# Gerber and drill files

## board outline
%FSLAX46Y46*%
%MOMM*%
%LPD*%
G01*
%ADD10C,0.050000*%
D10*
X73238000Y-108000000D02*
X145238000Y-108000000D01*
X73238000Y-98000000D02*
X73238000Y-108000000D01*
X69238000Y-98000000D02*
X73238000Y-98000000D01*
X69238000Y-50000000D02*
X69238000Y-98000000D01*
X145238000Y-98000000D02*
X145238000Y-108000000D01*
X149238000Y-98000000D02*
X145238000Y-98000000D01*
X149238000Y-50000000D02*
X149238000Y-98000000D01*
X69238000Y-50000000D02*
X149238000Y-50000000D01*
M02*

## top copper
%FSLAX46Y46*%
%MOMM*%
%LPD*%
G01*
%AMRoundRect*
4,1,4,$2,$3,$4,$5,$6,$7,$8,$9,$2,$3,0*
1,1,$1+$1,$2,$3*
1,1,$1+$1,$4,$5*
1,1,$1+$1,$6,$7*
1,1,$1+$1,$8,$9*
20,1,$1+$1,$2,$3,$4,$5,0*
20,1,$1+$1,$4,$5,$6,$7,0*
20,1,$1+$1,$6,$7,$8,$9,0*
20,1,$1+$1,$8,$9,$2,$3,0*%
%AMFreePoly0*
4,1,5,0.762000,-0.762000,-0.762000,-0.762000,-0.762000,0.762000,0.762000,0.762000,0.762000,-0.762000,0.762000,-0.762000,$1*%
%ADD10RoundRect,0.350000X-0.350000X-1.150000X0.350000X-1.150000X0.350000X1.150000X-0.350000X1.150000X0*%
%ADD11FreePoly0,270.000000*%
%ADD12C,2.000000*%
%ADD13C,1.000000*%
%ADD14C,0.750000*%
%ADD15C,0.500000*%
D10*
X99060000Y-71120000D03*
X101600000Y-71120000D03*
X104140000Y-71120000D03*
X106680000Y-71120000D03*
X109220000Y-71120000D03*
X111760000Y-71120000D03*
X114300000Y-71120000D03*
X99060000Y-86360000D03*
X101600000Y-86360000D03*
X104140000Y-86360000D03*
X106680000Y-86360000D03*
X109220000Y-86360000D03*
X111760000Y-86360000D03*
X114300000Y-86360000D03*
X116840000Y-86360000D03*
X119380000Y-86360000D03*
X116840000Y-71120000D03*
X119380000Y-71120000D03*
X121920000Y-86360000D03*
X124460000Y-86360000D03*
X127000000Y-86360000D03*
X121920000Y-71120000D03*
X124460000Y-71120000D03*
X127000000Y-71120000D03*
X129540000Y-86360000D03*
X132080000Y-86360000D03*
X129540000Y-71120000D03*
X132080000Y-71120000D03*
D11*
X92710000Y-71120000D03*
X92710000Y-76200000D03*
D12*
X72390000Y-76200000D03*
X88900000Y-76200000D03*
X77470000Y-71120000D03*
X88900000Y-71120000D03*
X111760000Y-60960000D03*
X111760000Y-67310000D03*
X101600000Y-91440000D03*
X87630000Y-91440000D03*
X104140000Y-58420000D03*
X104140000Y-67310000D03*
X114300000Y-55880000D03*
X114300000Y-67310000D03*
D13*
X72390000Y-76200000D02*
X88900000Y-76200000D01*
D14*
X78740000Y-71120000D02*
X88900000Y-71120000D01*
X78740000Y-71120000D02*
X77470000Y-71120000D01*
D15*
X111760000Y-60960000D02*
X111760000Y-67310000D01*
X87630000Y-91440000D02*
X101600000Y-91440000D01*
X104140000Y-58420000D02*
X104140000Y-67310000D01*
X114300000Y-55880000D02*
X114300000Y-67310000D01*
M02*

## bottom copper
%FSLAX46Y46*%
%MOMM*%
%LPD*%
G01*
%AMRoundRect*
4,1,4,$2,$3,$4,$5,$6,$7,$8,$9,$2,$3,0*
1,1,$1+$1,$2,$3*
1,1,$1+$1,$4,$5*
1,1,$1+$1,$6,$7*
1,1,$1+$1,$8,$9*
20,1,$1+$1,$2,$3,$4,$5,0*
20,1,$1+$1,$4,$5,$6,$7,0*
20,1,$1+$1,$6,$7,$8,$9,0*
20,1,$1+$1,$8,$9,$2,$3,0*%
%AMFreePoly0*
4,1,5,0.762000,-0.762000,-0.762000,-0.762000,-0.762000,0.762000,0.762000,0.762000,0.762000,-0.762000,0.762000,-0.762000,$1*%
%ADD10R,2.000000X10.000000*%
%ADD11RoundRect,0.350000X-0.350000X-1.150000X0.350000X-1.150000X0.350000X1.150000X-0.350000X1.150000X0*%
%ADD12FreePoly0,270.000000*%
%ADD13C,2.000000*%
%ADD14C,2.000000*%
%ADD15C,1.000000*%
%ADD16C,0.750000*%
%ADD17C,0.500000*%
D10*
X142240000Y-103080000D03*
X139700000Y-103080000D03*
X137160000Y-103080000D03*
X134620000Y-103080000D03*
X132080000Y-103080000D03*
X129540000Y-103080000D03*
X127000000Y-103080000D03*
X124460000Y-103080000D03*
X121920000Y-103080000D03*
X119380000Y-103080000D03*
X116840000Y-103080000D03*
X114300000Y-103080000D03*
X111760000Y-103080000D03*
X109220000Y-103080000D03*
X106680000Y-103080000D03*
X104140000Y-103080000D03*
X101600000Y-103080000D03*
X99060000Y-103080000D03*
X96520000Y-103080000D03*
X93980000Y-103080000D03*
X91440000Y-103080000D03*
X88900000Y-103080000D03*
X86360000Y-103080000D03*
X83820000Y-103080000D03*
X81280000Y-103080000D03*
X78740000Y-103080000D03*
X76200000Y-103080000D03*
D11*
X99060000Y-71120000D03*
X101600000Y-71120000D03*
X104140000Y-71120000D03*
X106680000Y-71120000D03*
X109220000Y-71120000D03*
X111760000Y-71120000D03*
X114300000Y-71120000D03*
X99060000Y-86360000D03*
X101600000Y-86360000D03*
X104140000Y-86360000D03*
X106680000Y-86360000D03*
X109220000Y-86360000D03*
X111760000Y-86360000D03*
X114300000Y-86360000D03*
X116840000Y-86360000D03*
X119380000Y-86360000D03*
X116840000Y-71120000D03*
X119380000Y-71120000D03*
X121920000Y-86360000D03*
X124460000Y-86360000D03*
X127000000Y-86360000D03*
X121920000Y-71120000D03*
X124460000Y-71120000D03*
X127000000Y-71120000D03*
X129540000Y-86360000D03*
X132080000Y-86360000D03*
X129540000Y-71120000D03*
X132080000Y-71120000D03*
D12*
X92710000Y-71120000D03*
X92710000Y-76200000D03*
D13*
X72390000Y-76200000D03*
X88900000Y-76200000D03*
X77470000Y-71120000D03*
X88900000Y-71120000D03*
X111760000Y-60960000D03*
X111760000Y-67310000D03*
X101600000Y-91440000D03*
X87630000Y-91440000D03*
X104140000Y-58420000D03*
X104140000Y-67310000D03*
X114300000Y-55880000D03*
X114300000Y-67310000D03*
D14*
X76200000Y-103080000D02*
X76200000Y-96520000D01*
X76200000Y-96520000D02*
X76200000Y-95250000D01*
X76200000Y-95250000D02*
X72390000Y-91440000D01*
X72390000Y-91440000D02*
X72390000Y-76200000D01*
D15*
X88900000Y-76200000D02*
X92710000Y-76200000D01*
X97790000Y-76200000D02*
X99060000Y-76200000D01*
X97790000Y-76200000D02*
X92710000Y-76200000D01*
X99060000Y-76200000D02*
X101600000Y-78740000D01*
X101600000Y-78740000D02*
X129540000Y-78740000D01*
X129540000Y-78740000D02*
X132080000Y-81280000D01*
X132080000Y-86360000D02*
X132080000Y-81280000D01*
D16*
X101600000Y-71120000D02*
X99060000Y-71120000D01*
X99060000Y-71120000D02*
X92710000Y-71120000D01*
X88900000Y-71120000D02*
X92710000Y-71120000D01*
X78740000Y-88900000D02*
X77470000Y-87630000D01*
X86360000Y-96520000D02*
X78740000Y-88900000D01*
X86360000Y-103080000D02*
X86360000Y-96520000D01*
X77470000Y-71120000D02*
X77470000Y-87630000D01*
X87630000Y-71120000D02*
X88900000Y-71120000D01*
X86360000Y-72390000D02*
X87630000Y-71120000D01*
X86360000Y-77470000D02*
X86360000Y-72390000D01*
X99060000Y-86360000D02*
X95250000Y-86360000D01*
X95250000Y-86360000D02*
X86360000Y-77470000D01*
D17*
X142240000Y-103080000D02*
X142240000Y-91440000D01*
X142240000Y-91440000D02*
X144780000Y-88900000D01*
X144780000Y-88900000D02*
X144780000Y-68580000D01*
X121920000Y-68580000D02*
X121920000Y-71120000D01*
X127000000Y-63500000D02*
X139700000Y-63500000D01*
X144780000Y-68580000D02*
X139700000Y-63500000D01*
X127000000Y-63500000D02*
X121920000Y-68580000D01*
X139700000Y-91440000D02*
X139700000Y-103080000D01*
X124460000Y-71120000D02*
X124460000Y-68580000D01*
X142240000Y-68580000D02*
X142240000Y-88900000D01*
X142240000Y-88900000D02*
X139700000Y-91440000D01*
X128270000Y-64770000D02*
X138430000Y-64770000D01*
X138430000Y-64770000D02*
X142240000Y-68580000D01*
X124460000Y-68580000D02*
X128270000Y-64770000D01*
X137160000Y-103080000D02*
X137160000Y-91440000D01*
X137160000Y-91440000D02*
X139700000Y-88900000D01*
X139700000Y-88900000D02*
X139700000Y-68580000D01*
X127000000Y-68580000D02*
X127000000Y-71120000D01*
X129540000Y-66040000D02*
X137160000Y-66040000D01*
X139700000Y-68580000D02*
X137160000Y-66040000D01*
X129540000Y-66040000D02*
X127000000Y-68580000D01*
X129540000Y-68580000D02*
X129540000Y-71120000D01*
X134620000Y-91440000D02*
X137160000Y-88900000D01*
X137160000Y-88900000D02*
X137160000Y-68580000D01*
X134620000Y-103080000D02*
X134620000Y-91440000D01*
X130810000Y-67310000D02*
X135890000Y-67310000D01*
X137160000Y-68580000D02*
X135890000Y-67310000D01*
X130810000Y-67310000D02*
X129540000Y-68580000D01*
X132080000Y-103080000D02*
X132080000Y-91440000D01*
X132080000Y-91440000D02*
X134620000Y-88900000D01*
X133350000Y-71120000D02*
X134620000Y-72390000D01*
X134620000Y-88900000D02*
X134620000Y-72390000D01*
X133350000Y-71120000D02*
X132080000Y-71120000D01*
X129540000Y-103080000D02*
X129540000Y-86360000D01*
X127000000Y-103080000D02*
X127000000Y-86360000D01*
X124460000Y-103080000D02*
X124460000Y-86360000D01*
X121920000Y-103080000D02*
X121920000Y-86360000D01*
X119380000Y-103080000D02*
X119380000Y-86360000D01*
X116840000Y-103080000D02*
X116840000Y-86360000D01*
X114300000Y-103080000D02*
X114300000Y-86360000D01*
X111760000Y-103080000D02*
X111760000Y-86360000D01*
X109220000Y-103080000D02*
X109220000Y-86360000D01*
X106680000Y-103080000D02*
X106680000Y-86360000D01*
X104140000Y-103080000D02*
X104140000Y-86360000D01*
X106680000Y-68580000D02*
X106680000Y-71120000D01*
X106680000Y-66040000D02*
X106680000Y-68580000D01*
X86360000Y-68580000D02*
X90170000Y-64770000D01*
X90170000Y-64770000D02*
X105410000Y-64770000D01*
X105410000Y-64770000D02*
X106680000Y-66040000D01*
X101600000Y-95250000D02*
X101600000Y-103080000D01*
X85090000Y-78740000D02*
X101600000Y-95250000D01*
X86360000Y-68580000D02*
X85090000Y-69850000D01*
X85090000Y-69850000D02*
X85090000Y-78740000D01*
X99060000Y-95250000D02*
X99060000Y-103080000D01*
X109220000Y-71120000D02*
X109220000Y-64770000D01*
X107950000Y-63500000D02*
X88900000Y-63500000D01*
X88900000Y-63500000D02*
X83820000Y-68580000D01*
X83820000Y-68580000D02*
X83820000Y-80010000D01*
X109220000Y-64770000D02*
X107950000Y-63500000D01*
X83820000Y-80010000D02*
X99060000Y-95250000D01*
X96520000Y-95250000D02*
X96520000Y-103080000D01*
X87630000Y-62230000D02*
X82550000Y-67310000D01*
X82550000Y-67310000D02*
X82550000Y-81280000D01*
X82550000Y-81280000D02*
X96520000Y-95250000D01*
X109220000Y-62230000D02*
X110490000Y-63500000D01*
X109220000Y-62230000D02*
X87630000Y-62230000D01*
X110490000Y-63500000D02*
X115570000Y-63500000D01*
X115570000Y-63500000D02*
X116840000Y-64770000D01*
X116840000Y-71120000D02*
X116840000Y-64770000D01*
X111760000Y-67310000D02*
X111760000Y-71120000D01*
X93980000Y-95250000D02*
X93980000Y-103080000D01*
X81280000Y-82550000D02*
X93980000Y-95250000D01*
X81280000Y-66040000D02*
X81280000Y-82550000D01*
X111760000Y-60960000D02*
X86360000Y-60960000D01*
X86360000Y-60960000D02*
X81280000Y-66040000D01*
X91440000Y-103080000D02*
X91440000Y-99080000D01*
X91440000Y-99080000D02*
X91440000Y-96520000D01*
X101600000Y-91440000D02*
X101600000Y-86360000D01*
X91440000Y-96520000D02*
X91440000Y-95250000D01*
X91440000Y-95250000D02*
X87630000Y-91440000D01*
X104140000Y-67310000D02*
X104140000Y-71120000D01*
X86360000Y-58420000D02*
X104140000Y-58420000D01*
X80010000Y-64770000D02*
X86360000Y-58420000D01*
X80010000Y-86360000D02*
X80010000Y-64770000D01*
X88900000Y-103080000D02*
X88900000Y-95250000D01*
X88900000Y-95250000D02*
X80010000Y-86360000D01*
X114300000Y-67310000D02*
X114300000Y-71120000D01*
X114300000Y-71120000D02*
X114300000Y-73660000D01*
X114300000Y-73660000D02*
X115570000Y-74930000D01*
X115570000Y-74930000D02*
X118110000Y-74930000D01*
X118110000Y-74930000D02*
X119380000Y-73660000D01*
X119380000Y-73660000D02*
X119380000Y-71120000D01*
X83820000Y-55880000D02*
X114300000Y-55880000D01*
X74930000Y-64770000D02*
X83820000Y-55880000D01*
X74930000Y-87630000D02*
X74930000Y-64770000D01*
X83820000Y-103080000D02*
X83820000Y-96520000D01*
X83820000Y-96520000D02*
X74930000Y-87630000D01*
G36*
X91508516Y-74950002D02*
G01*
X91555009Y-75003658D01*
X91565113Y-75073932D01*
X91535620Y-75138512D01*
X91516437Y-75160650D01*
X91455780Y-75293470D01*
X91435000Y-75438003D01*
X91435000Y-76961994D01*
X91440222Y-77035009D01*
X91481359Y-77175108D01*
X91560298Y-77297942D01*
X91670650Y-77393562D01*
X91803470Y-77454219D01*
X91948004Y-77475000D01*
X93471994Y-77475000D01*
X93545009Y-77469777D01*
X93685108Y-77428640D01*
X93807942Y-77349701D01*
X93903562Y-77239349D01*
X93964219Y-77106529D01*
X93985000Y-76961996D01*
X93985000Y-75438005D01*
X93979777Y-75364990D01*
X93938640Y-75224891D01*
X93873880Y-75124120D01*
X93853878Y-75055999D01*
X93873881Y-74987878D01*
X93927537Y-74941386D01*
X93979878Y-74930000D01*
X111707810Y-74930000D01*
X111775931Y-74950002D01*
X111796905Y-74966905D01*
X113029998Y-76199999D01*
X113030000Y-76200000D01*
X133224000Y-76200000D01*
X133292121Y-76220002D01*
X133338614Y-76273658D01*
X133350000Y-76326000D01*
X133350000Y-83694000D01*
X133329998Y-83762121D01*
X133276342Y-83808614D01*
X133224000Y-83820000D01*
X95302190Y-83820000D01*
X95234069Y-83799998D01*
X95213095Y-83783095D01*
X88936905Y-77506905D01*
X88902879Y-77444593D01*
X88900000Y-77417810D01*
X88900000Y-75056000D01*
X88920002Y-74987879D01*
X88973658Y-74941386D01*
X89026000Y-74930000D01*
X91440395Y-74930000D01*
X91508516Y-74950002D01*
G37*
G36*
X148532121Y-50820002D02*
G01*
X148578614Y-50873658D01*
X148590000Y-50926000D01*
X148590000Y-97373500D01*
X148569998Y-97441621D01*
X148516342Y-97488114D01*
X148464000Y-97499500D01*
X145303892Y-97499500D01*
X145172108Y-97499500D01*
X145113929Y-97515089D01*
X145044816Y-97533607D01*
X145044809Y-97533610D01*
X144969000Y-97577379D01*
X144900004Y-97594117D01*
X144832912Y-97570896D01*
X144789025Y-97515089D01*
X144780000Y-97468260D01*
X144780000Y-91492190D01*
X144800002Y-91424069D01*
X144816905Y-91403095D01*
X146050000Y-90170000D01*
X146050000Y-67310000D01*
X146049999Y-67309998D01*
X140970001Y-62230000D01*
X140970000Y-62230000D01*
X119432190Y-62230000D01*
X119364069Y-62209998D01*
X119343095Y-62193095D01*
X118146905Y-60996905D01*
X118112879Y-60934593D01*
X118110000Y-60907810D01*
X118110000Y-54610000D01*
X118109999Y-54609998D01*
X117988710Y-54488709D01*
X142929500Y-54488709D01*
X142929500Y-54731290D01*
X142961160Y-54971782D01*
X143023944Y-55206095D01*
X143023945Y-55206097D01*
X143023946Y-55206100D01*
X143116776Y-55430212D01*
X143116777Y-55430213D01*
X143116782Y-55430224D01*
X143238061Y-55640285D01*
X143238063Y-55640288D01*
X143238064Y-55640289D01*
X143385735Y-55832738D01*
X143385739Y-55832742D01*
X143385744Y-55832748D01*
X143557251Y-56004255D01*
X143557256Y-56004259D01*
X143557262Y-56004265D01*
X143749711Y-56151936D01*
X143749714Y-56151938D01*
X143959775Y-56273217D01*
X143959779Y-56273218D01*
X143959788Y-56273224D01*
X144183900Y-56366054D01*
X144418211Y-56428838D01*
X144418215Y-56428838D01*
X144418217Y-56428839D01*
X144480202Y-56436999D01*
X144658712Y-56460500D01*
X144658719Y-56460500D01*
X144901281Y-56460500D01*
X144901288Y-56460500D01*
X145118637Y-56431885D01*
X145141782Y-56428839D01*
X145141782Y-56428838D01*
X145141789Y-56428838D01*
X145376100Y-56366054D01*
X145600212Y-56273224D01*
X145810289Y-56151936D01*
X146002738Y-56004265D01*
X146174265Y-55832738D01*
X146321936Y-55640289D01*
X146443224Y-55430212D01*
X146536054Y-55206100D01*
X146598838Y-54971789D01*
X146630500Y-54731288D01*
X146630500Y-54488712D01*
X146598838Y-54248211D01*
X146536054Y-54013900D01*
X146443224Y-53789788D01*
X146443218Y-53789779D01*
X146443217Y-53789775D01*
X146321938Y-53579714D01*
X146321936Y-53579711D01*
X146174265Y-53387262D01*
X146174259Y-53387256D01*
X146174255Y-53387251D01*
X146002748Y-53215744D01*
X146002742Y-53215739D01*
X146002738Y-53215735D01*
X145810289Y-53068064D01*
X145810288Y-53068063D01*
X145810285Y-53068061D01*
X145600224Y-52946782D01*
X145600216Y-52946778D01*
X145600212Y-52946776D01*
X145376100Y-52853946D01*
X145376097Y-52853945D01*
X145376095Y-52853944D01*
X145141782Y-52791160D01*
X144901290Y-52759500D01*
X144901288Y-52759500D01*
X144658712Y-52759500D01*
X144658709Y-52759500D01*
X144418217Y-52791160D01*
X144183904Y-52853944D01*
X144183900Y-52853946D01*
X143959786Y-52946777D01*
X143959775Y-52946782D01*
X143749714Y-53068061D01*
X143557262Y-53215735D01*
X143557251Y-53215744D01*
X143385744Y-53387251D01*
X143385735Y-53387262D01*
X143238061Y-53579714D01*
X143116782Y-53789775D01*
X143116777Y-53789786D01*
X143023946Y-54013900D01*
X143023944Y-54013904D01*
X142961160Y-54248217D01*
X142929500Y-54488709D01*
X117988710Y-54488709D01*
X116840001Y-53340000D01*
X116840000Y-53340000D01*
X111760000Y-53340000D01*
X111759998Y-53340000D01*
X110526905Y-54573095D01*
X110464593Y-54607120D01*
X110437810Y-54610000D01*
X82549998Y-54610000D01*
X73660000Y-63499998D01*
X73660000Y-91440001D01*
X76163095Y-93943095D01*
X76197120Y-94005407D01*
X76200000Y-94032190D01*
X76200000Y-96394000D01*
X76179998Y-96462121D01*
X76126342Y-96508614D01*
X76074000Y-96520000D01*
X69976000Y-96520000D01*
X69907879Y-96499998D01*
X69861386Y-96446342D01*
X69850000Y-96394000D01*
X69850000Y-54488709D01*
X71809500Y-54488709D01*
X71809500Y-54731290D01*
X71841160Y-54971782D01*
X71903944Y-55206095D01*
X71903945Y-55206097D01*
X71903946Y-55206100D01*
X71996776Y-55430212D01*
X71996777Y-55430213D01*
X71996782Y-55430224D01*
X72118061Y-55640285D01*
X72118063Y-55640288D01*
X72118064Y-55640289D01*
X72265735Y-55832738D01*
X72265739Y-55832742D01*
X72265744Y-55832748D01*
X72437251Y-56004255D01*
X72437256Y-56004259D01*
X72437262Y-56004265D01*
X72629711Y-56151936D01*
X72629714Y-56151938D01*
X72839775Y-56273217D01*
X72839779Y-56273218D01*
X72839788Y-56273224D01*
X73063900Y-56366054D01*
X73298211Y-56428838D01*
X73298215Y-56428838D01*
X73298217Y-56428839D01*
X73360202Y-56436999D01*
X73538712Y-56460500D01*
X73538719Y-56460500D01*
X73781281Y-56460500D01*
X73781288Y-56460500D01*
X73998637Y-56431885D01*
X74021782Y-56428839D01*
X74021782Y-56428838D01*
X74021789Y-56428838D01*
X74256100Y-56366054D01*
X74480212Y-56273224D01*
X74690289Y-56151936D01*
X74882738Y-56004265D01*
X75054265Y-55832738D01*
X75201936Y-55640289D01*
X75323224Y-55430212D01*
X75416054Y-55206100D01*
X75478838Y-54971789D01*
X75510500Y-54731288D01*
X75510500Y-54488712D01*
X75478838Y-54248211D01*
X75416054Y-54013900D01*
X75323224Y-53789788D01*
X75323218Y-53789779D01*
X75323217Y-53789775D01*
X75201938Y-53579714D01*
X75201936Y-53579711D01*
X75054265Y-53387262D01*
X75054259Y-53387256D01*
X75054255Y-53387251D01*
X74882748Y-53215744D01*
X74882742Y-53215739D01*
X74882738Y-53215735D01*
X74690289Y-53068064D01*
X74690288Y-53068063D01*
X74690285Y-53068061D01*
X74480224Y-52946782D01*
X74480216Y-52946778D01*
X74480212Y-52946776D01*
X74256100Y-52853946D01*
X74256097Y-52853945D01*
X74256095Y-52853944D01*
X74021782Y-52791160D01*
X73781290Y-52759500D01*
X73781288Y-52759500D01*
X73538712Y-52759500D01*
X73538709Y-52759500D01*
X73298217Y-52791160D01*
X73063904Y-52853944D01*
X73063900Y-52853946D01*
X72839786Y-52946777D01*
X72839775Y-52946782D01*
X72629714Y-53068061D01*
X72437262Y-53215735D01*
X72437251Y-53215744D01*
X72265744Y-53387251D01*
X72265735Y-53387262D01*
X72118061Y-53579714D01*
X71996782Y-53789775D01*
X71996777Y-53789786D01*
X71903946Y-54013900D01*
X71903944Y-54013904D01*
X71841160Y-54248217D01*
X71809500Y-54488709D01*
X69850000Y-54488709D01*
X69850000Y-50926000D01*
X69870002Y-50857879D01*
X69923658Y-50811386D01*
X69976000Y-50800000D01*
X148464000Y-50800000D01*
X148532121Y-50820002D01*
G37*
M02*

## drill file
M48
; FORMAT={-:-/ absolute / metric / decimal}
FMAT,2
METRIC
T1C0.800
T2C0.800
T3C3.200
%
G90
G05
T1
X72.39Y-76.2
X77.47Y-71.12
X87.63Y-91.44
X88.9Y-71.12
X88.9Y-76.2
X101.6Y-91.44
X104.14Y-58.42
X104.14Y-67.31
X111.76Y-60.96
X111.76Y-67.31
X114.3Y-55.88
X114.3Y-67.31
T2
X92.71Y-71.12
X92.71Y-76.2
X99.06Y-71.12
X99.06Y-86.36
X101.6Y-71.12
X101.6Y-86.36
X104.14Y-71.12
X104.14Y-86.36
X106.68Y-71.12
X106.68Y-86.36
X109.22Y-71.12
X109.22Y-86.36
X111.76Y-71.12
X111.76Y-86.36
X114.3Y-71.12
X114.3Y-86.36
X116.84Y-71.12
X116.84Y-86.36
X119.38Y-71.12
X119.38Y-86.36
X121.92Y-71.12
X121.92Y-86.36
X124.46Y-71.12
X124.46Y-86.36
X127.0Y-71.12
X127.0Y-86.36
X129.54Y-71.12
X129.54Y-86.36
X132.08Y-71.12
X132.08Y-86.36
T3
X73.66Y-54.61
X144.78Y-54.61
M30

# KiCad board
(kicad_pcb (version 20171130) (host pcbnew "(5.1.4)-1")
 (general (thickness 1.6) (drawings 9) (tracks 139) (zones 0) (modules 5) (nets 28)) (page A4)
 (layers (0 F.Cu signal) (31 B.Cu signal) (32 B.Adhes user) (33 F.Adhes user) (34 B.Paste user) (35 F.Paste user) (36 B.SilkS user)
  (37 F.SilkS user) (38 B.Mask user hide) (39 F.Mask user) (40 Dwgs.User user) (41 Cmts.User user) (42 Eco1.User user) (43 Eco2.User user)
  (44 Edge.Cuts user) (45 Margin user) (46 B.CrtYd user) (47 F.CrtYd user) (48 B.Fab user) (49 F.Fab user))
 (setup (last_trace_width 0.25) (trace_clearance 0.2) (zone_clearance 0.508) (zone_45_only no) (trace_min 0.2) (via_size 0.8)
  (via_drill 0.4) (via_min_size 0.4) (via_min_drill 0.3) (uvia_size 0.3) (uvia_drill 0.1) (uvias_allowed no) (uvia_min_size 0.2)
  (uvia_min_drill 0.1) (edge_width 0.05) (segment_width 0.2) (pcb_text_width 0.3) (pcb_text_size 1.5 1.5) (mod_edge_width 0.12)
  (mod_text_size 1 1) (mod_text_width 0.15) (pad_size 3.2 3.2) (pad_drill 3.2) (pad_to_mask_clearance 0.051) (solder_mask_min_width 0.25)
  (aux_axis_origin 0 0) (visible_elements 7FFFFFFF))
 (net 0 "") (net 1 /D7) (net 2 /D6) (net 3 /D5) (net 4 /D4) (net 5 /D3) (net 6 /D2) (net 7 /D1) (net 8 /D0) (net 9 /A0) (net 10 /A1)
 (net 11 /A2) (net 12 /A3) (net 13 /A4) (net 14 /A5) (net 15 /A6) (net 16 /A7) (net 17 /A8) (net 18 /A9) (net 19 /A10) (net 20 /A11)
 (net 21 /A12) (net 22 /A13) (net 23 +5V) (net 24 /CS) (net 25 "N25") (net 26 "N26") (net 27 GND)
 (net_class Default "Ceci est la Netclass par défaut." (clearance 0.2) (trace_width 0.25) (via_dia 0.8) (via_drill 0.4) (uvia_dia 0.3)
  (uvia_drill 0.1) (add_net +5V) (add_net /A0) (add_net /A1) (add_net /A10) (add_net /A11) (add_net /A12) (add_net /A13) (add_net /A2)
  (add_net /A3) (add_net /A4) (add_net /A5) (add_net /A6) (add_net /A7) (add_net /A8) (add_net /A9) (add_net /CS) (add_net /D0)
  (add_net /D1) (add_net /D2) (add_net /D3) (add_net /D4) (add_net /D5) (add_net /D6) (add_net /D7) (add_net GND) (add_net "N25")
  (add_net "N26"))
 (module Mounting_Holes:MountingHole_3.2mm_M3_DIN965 (layer F.Cu) (at 73.66 54.61)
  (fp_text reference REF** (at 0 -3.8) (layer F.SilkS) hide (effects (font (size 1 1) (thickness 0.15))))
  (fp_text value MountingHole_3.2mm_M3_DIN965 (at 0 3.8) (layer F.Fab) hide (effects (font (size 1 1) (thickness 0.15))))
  (pad "" np_thru_hole circle (at 0 0) (size 3.2 3.2) (drill 3.2) (layers *.Cu *.Mask)))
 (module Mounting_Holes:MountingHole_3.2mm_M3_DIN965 (layer F.Cu) (at 144.78 54.61)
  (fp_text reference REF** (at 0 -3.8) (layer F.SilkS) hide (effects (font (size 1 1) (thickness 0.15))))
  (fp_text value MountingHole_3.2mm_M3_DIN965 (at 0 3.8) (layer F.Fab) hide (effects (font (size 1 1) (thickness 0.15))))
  (pad "" np_thru_hole circle (at 0 0) (size 3.2 3.2) (drill 3.2) (layers *.Cu *.Mask)))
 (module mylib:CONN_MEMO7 (layer B.Cu) (at 106.68 98 180)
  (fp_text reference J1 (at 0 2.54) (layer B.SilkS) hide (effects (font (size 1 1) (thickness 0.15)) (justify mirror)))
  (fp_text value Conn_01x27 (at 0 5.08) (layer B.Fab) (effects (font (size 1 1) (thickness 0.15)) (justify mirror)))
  (pad 1 connect rect (at -35.56 -5.08 180) (size 2 10) (layers B.Cu B.Mask) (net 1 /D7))
  (pad 2 connect rect (at -33.02 -5.08 180) (size 2 10) (layers B.Cu B.Mask) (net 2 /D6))
  (pad 3 connect rect (at -30.48 -5.08 180) (size 2 10) (layers B.Cu B.Mask) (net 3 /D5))
  (pad 4 connect rect (at -27.94 -5.08 180) (size 2 10) (layers B.Cu B.Mask) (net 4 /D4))
  (pad 5 connect rect (at -25.4 -5.08 180) (size 2 10) (layers B.Cu B.Mask) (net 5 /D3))
  (pad 6 connect rect (at -22.86 -5.08 180) (size 2 10) (layers B.Cu B.Mask) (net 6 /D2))
  (pad 7 connect rect (at -20.32 -5.08 180) (size 2 10) (layers B.Cu B.Mask) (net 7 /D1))
  (pad 8 connect rect (at -17.78 -5.08 180) (size 2 10) (layers B.Cu B.Mask) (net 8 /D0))
  (pad 9 connect rect (at -15.24 -5.08 180) (size 2 10) (layers B.Cu B.Mask) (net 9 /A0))
  (pad 10 connect rect (at -12.7 -5.08 180) (size 2 10) (layers B.Cu B.Mask) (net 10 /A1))
  (pad 11 connect rect (at -10.16 -5.08 180) (size 2 10) (layers B.Cu B.Mask) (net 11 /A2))
  (pad 12 connect rect (at -7.62 -5.08 180) (size 2 10) (layers B.Cu B.Mask) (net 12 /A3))
  (pad 13 connect rect (at -5.08 -5.08 180) (size 2 10) (layers B.Cu B.Mask) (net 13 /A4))
  (pad 14 connect rect (at -2.54 -5.08 180) (size 2 10) (layers B.Cu B.Mask) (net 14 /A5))
  (pad 15 connect rect (at 0 -5.08 180) (size 2 10) (layers B.Cu B.Mask) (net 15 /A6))
  (pad 16 connect rect (at 2.54 -5.08 180) (size 2 10) (layers B.Cu B.Mask) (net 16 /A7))
  (pad 17 connect rect (at 5.08 -5.08 180) (size 2 10) (layers B.Cu B.Mask) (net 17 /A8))
  (pad 18 connect rect (at 7.62 -5.08 180) (size 2 10) (layers B.Cu B.Mask) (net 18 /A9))
  (pad 19 connect rect (at 10.16 -5.08 180) (size 2 10) (layers B.Cu B.Mask) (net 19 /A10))
  (pad 20 connect rect (at 12.7 -5.08 180) (size 2 10) (layers B.Cu B.Mask) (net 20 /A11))
  (pad 21 connect rect (at 15.24 -5.08 180) (size 2 10) (layers B.Cu B.Mask) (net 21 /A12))
  (pad 22 connect rect (at 17.78 -5.08 180) (size 2 10) (layers B.Cu B.Mask) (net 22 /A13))
  (pad 23 connect rect (at 20.32 -5.08 180) (size 2 10) (layers B.Cu B.Mask) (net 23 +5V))
  (pad 24 connect rect (at 22.86 -5.08 180) (size 2 10) (layers B.Cu B.Mask) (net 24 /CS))
  (pad 25 connect rect (at 25.4 -5.08 180) (size 2 10) (layers B.Cu B.Mask) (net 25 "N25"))
  (pad 26 connect rect (at 27.94 -5.08 180) (size 2 10) (layers B.Cu B.Mask) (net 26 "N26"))
  (pad 27 connect rect (at 30.48 -5.08 180) (size 2 10) (layers B.Cu B.Mask) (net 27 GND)))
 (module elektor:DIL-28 (layer F.Cu) (at 113.03 78.74)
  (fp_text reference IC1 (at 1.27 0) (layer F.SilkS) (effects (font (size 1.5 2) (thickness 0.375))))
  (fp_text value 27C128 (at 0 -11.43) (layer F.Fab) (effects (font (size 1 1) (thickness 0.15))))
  (pad 28 thru_hole roundrect (at -13.97 -7.62) (size 1.4 3) (drill 0.8) (layers *.Cu *.Mask) (roundrect_rratio 0.25) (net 23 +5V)
   (zone_connect 0))
  (pad 27 thru_hole roundrect (at -11.43 -7.62) (size 1.4 3) (drill 0.8) (layers *.Cu *.Mask) (roundrect_rratio 0.25) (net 23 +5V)
   (zone_connect 0))
  (pad 26 thru_hole roundrect (at -8.89 -7.62) (size 1.4 3) (drill 0.8) (layers *.Cu *.Mask) (roundrect_rratio 0.25) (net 22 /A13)
   (zone_connect 0))
  (pad 25 thru_hole roundrect (at -6.35 -7.62) (size 1.4 3) (drill 0.8) (layers *.Cu *.Mask) (roundrect_rratio 0.25) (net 17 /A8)
   (zone_connect 0))
  (pad 24 thru_hole roundrect (at -3.81 -7.62) (size 1.4 3) (drill 0.8) (layers *.Cu *.Mask) (roundrect_rratio 0.25) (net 18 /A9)
   (zone_connect 0))
  (pad 23 thru_hole roundrect (at -1.27 -7.62) (size 1.4 3) (drill 0.8) (layers *.Cu *.Mask) (roundrect_rratio 0.25) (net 20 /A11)
   (zone_connect 0))
  (pad 22 thru_hole roundrect (at 1.27 -7.62) (size 1.4 3) (drill 0.8) (layers *.Cu *.Mask) (roundrect_rratio 0.25) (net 24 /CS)
   (zone_connect 0))
  (pad 1 thru_hole roundrect (at -13.97 7.62) (size 1.4 3) (drill 0.8) (layers *.Cu *.Mask) (roundrect_rratio 0.25) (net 23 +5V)
   (zone_connect 0))
  (pad 2 thru_hole roundrect (at -11.43 7.62) (size 1.4 3) (drill 0.8) (layers *.Cu *.Mask) (roundrect_rratio 0.25) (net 21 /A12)
   (zone_connect 0))
  (pad 3 thru_hole roundrect (at -8.89 7.62) (size 1.4 3) (drill 0.8) (layers *.Cu *.Mask) (roundrect_rratio 0.25) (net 16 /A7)
   (zone_connect 0))
  (pad 4 thru_hole roundrect (at -6.35 7.62) (size 1.4 3) (drill 0.8) (layers *.Cu *.Mask) (roundrect_rratio 0.25) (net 15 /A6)
   (zone_connect 0))
  (pad 5 thru_hole roundrect (at -3.81 7.62) (size 1.4 3) (drill 0.8) (layers *.Cu *.Mask) (roundrect_rratio 0.25) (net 14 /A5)
   (zone_connect 0))
  (pad 6 thru_hole roundrect (at -1.27 7.62) (size 1.4 3) (drill 0.8) (layers *.Cu *.Mask) (roundrect_rratio 0.25) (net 13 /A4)
   (zone_connect 0))
  (pad 7 thru_hole roundrect (at 1.27 7.62) (size 1.4 3) (drill 0.8) (layers *.Cu *.Mask) (roundrect_rratio 0.25) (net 12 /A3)
   (zone_connect 0))
  (pad 8 thru_hole roundrect (at 3.81 7.62) (size 1.4 3) (drill 0.8) (layers *.Cu *.Mask) (roundrect_rratio 0.25) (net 11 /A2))
  (pad 9 thru_hole roundrect (at 6.35 7.62) (size 1.4 3) (drill 0.8) (layers *.Cu *.Mask) (roundrect_rratio 0.25) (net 10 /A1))
  (pad 21 thru_hole roundrect (at 3.81 -7.62) (size 1.4 3) (drill 0.8) (layers *.Cu *.Mask) (roundrect_rratio 0.25) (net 19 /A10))
  (pad 20 thru_hole roundrect (at 6.35 -7.62) (size 1.4 3) (drill 0.8) (layers *.Cu *.Mask) (roundrect_rratio 0.25) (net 24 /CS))
  (pad 10 thru_hole roundrect (at 8.89 7.62) (size 1.4 3) (drill 0.8) (layers *.Cu *.Mask) (roundrect_rratio 0.25) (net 9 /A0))
  (pad 11 thru_hole roundrect (at 11.43 7.62) (size 1.4 3) (drill 0.8) (layers *.Cu *.Mask) (roundrect_rratio 0.25) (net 8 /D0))
  (pad 12 thru_hole roundrect (at 13.97 7.62) (size 1.4 3) (drill 0.8) (layers *.Cu *.Mask) (roundrect_rratio 0.25) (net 7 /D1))
  (pad 19 thru_hole roundrect (at 8.89 -7.62) (size 1.4 3) (drill 0.8) (layers *.Cu *.Mask) (roundrect_rratio 0.25) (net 1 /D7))
  (pad 18 thru_hole roundrect (at 11.43 -7.62) (size 1.4 3) (drill 0.8) (layers *.Cu *.Mask) (roundrect_rratio 0.25) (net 2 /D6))
  (pad 17 thru_hole roundrect (at 13.97 -7.62) (size 1.4 3) (drill 0.8) (layers *.Cu *.Mask) (roundrect_rratio 0.25) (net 3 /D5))
  (pad 13 thru_hole roundrect (at 16.51 7.62) (size 1.4 3) (drill 0.8) (layers *.Cu *.Mask) (roundrect_rratio 0.25) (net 6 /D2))
  (pad 14 thru_hole roundrect (at 19.05 7.62) (size 1.4 3) (drill 0.8) (layers *.Cu *.Mask) (roundrect_rratio 0.25) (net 27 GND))
  (pad 16 thru_hole roundrect (at 16.51 -7.62) (size 1.4 3) (drill 0.8) (layers *.Cu *.Mask) (roundrect_rratio 0.25) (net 4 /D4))
  (pad 15 thru_hole roundrect (at 19.05 -7.62) (size 1.4 3) (drill 0.8) (layers *.Cu *.Mask) (roundrect_rratio 0.25) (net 5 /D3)))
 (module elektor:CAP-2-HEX (layer F.Cu) (at 92.71 73.66 270)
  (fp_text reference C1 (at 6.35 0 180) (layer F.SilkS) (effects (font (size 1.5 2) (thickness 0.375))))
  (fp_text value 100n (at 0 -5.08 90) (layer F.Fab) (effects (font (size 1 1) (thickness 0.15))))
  (pad 1 thru_hole custom (at -2.54 0 270) (size 1.524 1.524) (drill 0.8) (layers *.Cu *.Mask) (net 23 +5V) (zone_connect 0)
   (options (clearance outline) (anchor rect)) (primitives))
  (pad 2 thru_hole custom (at 2.54 0 270) (size 1.524 1.524) (drill 0.8) (layers *.Cu *.Mask) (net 27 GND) (zone_connect 0)
   (options (clearance outline) (anchor rect)) (primitives)))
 (gr_line (start 73.238 108) (end 145.238 108) (layer Edge.Cuts) (width 0.05))
 (gr_line (start 73.238 98) (end 73.238 108) (layer Edge.Cuts) (width 0.05))
 (gr_line (start 69.238 98) (end 73.238 98) (layer Edge.Cuts) (width 0.05))
 (gr_line (start 69.238 50) (end 69.238 98) (layer Edge.Cuts) (width 0.05))
 (gr_line (start 145.238 98) (end 145.238 108) (layer Edge.Cuts) (width 0.05))
 (gr_line (start 149.238 98) (end 145.238 98) (layer Edge.Cuts) (width 0.05))
 (gr_line (start 149.238 50) (end 149.238 98) (layer Edge.Cuts) (width 0.05))
 (gr_line (start 69.238 50) (end 149.238 50) (layer Edge.Cuts) (width 0.05))
 (segment (start 76.2 103.08) (end 76.2 96.52) (width 2) (layer B.Cu) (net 27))
 (segment (start 76.2 96.52) (end 76.2 95.25) (width 2) (layer B.Cu) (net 27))
 (via (at 72.39 76.2) (size 2) (drill 0.8) (layers F.Cu B.Cu) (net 27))
 (segment (start 76.2 95.25) (end 72.39 91.44) (width 2) (layer B.Cu) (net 27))
 (segment (start 72.39 91.44) (end 72.39 76.2) (width 2) (layer B.Cu) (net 27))
 (via (at 88.9 76.2) (size 2) (drill 0.8) (layers F.Cu B.Cu) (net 27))
 (segment (start 72.39 76.2) (end 88.9 76.2) (width 1) (layer F.Cu) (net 27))
 (segment (start 88.9 76.2) (end 92.71 76.2) (width 1) (layer B.Cu) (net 27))
 (segment (start 97.79 76.2) (end 99.06 76.2) (width 1) (layer B.Cu) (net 27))
 (segment (start 97.79 76.2) (end 92.71 76.2) (width 1) (layer B.Cu) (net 27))
 (segment (start 99.06 76.2) (end 101.6 78.74) (width 1) (layer B.Cu) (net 27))
 (segment (start 101.6 78.74) (end 129.54 78.74) (width 1) (layer B.Cu) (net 27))
 (segment (start 129.54 78.74) (end 132.08 81.28) (width 1) (layer B.Cu) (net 27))
 (segment (start 132.08 86.36) (end 132.08 81.28) (width 1) (layer B.Cu) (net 27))
 (segment (start 101.6 71.12) (end 99.06 71.12) (width 0.75) (layer B.Cu) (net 23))
 (segment (start 99.06 71.12) (end 92.71 71.12) (width 0.75) (layer B.Cu) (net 23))
 (via (at 77.47 71.12) (size 2) (drill 0.8) (layers F.Cu B.Cu) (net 23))
 (via (at 88.9 71.12) (size 2) (drill 0.8) (layers F.Cu B.Cu) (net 23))
 (segment (start 78.74 71.12) (end 88.9 71.12) (width 0.75) (layer F.Cu) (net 23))
 (segment (start 88.9 71.12) (end 92.71 71.12) (width 0.75) (layer B.Cu) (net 23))
 (segment (start 78.74 71.12) (end 77.47 71.12) (width 0.75) (layer F.Cu) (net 23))
 (segment (start 78.74 88.9) (end 77.47 87.63) (width 0.75) (layer B.Cu) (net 23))
 (segment (start 86.36 96.52) (end 78.74 88.9) (width 0.75) (layer B.Cu) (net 23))
 (segment (start 86.36 103.08) (end 86.36 96.52) (width 0.75) (layer B.Cu) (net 23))
 (segment (start 77.47 71.12) (end 77.47 87.63) (width 0.75) (layer B.Cu) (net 23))
 (segment (start 87.63 71.12) (end 88.9 71.12) (width 0.75) (layer B.Cu) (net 23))
 (segment (start 86.36 72.39) (end 87.63 71.12) (width 0.75) (layer B.Cu) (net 23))
 (segment (start 86.36 77.47) (end 86.36 72.39) (width 0.75) (layer B.Cu) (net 23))
 (segment (start 99.06 86.36) (end 95.25 86.36) (width 0.75) (layer B.Cu) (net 23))
 (segment (start 95.25 86.36) (end 86.36 77.47) (width 0.75) (layer B.Cu) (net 23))
 (segment (start 142.24 103.08) (end 142.24 91.44) (width 0.5) (layer B.Cu) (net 1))
 (segment (start 142.24 91.44) (end 144.78 88.9) (width 0.5) (layer B.Cu) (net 1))
 (segment (start 144.78 88.9) (end 144.78 68.58) (width 0.5) (layer B.Cu) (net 1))
 (segment (start 121.92 68.58) (end 121.92 71.12) (width 0.5) (layer B.Cu) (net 1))
 (segment (start 127 63.5) (end 139.7 63.5) (width 0.5) (layer B.Cu) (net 1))
 (segment (start 144.78 68.58) (end 139.7 63.5) (width 0.5) (layer B.Cu) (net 1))
 (segment (start 127 63.5) (end 121.92 68.58) (width 0.5) (layer B.Cu) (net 1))
 (segment (start 139.7 91.44) (end 139.7 103.08) (width 0.5) (layer B.Cu) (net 2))
 (segment (start 124.46 71.12) (end 124.46 68.58) (width 0.5) (layer B.Cu) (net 2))
 (segment (start 142.24 68.58) (end 142.24 88.9) (width 0.5) (layer B.Cu) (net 2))
 (segment (start 142.24 88.9) (end 139.7 91.44) (width 0.5) (layer B.Cu) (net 2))
 (segment (start 128.27 64.77) (end 138.43 64.77) (width 0.5) (layer B.Cu) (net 2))
 (segment (start 138.43 64.77) (end 142.24 68.58) (width 0.5) (layer B.Cu) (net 2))
 (segment (start 124.46 68.58) (end 128.27 64.77) (width 0.5) (layer B.Cu) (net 2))
 (segment (start 137.16 103.08) (end 137.16 91.44) (width 0.5) (layer B.Cu) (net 3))
 (segment (start 137.16 91.44) (end 139.7 88.9) (width 0.5) (layer B.Cu) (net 3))
 (segment (start 139.7 88.9) (end 139.7 68.58) (width 0.5) (layer B.Cu) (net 3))
 (segment (start 127 68.58) (end 127 71.12) (width 0.5) (layer B.Cu) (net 3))
 (segment (start 129.54 66.04) (end 137.16 66.04) (width 0.5) (layer B.Cu) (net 3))
 (segment (start 139.7 68.58) (end 137.16 66.04) (width 0.5) (layer B.Cu) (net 3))
 (segment (start 129.54 66.04) (end 127 68.58) (width 0.5) (layer B.Cu) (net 3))
 (segment (start 129.54 68.58) (end 129.54 71.12) (width 0.5) (layer B.Cu) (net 4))
 (segment (start 134.62 91.44) (end 137.16 88.9) (width 0.5) (layer B.Cu) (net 4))
 (segment (start 137.16 88.9) (end 137.16 68.58) (width 0.5) (layer B.Cu) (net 4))
 (segment (start 134.62 103.08) (end 134.62 91.44) (width 0.5) (layer B.Cu) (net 4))
 (segment (start 130.81 67.31) (end 135.89 67.31) (width 0.5) (layer B.Cu) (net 4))
 (segment (start 137.16 68.58) (end 135.89 67.31) (width 0.5) (layer B.Cu) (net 4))
 (segment (start 130.81 67.31) (end 129.54 68.58) (width 0.5) (layer B.Cu) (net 4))
 (segment (start 132.08 103.08) (end 132.08 91.44) (width 0.5) (layer B.Cu) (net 5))
 (segment (start 132.08 91.44) (end 134.62 88.9) (width 0.5) (layer B.Cu) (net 5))
 (segment (start 133.35 71.12) (end 134.62 72.39) (width 0.5) (layer B.Cu) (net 5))
 (segment (start 134.62 88.9) (end 134.62 72.39) (width 0.5) (layer B.Cu) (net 5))
 (segment (start 133.35 71.12) (end 132.08 71.12) (width 0.5) (layer B.Cu) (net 5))
 (segment (start 129.54 103.08) (end 129.54 86.36) (width 0.5) (layer B.Cu) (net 6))
 (segment (start 127 103.08) (end 127 86.36) (width 0.5) (layer B.Cu) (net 7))
 (segment (start 124.46 103.08) (end 124.46 86.36) (width 0.5) (layer B.Cu) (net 8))
 (segment (start 121.92 103.08) (end 121.92 86.36) (width 0.5) (layer B.Cu) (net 9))
 (segment (start 119.38 103.08) (end 119.38 86.36) (width 0.5) (layer B.Cu) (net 10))
 (segment (start 116.84 103.08) (end 116.84 86.36) (width 0.5) (layer B.Cu) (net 11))
 (segment (start 114.3 103.08) (end 114.3 86.36) (width 0.5) (layer B.Cu) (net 12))
 (segment (start 111.76 103.08) (end 111.76 86.36) (width 0.5) (layer B.Cu) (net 13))
 (segment (start 109.22 103.08) (end 109.22 86.36) (width 0.5) (layer B.Cu) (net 14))
 (segment (start 106.68 103.08) (end 106.68 86.36) (width 0.5) (layer B.Cu) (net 15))
 (segment (start 104.14 103.08) (end 104.14 86.36) (width 0.5) (layer B.Cu) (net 16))
 (segment (start 106.68 68.58) (end 106.68 71.12) (width 0.5) (layer B.Cu) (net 17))
 (segment (start 106.68 66.04) (end 106.68 68.58) (width 0.5) (layer B.Cu) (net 17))
 (segment (start 86.36 68.58) (end 90.17 64.77) (width 0.5) (layer B.Cu) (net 17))
 (segment (start 90.17 64.77) (end 105.41 64.77) (width 0.5) (layer B.Cu) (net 17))
 (segment (start 105.41 64.77) (end 106.68 66.04) (width 0.5) (layer B.Cu) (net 17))
 (segment (start 101.6 95.25) (end 101.6 103.08) (width 0.5) (layer B.Cu) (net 17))
 (segment (start 85.09 78.74) (end 101.6 95.25) (width 0.5) (layer B.Cu) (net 17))
 (segment (start 86.36 68.58) (end 85.09 69.85) (width 0.5) (layer B.Cu) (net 17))
 (segment (start 85.09 69.85) (end 85.09 78.74) (width 0.5) (layer B.Cu) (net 17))
 (segment (start 99.06 95.25) (end 99.06 103.08) (width 0.5) (layer B.Cu) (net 18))
 (segment (start 109.22 71.12) (end 109.22 64.77) (width 0.5) (layer B.Cu) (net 18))
 (segment (start 107.95 63.5) (end 88.9 63.5) (width 0.5) (layer B.Cu) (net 18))
 (segment (start 88.9 63.5) (end 83.82 68.58) (width 0.5) (layer B.Cu) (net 18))
 (segment (start 83.82 68.58) (end 83.82 80.01) (width 0.5) (layer B.Cu) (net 18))
 (segment (start 109.22 64.77) (end 107.95 63.5) (width 0.5) (layer B.Cu) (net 18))
 (segment (start 83.82 80.01) (end 99.06 95.25) (width 0.5) (layer B.Cu) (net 18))
 (segment (start 96.52 95.25) (end 96.52 103.08) (width 0.5) (layer B.Cu) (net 19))
 (segment (start 87.63 62.23) (end 82.55 67.31) (width 0.5) (layer B.Cu) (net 19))
 (segment (start 82.55 67.31) (end 82.55 81.28) (width 0.5) (layer B.Cu) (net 19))
 (segment (start 82.55 81.28) (end 96.52 95.25) (width 0.5) (layer B.Cu) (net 19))
 (segment (start 109.22 62.23) (end 110.49 63.5) (width 0.5) (layer B.Cu) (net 19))
 (segment (start 109.22 62.23) (end 87.63 62.23) (width 0.5) (layer B.Cu) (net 19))
 (segment (start 110.49 63.5) (end 115.57 63.5) (width 0.5) (layer B.Cu) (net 19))
 (segment (start 115.57 63.5) (end 116.84 64.77) (width 0.5) (layer B.Cu) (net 19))
 (segment (start 116.84 71.12) (end 116.84 64.77) (width 0.5) (layer B.Cu) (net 19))
 (via (at 111.76 60.96) (size 2) (drill 0.8) (layers F.Cu B.Cu) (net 20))
 (via (at 111.76 67.31) (size 2) (drill 0.8) (layers F.Cu B.Cu) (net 20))
 (segment (start 111.76 60.96) (end 111.76 67.31) (width 0.5) (layer F.Cu) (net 20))
 (segment (start 111.76 67.31) (end 111.76 71.12) (width 0.5) (layer B.Cu) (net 20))
 (segment (start 93.98 95.25) (end 93.98 103.08) (width 0.5) (layer B.Cu) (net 20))
 (segment (start 81.28 82.55) (end 93.98 95.25) (width 0.5) (layer B.Cu) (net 20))
 (segment (start 81.28 66.04) (end 81.28 82.55) (width 0.5) (layer B.Cu) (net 20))
 (segment (start 111.76 60.96) (end 86.36 60.96) (width 0.5) (layer B.Cu) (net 20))
 (segment (start 86.36 60.96) (end 81.28 66.04) (width 0.5) (layer B.Cu) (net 20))
 (segment (start 91.44 103.08) (end 91.44 99.08) (width 0.5) (layer B.Cu) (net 21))
 (segment (start 91.44 99.08) (end 91.44 96.52) (width 0.5) (layer B.Cu) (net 21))
 (via (at 101.6 91.44) (size 2) (drill 0.8) (layers F.Cu B.Cu) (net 21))
 (segment (start 101.6 91.44) (end 101.6 86.36) (width 0.5) (layer B.Cu) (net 21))
 (segment (start 91.44 96.52) (end 91.44 95.25) (width 0.5) (layer B.Cu) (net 21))
 (via (at 87.63 91.44) (size 2) (drill 0.8) (layers F.Cu B.Cu) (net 21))
 (segment (start 91.44 95.25) (end 87.63 91.44) (width 0.5) (layer B.Cu) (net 21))
 (segment (start 87.63 91.44) (end 101.6 91.44) (width 0.5) (layer F.Cu) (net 21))
 (via (at 104.14 58.42) (size 2) (drill 0.8) (layers F.Cu B.Cu) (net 22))
 (via (at 104.14 67.31) (size 2) (drill 0.8) (layers F.Cu B.Cu) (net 22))
 (segment (start 104.14 58.42) (end 104.14 67.31) (width 0.5) (layer F.Cu) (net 22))
 (segment (start 104.14 67.31) (end 104.14 71.12) (width 0.5) (layer B.Cu) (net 22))
 (segment (start 86.36 58.42) (end 104.14 58.42) (width 0.5) (layer B.Cu) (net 22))
 (segment (start 80.01 64.77) (end 86.36 58.42) (width 0.5) (layer B.Cu) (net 22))
 (segment (start 80.01 86.36) (end 80.01 64.77) (width 0.5) (layer B.Cu) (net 22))
 (segment (start 88.9 103.08) (end 88.9 95.25) (width 0.5) (layer B.Cu) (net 22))
 (segment (start 88.9 95.25) (end 80.01 86.36) (width 0.5) (layer B.Cu) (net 22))
 (via (at 114.3 55.88) (size 2) (drill 0.8) (layers F.Cu B.Cu) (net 24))
 (via (at 114.3 67.31) (size 2) (drill 0.8) (layers F.Cu B.Cu) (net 24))
 (segment (start 114.3 55.88) (end 114.3 67.31) (width 0.5) (layer F.Cu) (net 24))
 (segment (start 114.3 67.31) (end 114.3 71.12) (width 0.5) (layer B.Cu) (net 24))
 (segment (start 114.3 71.12) (end 114.3 73.66) (width 0.5) (layer B.Cu) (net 24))
 (segment (start 114.3 73.66) (end 115.57 74.93) (width 0.5) (layer B.Cu) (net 24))
 (segment (start 115.57 74.93) (end 118.11 74.93) (width 0.5) (layer B.Cu) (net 24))
 (segment (start 118.11 74.93) (end 119.38 73.66) (width 0.5) (layer B.Cu) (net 24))
 (segment (start 119.38 73.66) (end 119.38 71.12) (width 0.5) (layer B.Cu) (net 24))
 (segment (start 83.82 55.88) (end 114.3 55.88) (width 0.5) (layer B.Cu) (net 24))
 (segment (start 74.93 64.77) (end 83.82 55.88) (width 0.5) (layer B.Cu) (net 24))
 (segment (start 74.93 87.63) (end 74.93 64.77) (width 0.5) (layer B.Cu) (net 24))
 (segment (start 83.82 103.08) (end 83.82 96.52) (width 0.5) (layer B.Cu) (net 24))
 (segment (start 83.82 96.52) (end 74.93 87.63) (width 0.5) (layer B.Cu) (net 24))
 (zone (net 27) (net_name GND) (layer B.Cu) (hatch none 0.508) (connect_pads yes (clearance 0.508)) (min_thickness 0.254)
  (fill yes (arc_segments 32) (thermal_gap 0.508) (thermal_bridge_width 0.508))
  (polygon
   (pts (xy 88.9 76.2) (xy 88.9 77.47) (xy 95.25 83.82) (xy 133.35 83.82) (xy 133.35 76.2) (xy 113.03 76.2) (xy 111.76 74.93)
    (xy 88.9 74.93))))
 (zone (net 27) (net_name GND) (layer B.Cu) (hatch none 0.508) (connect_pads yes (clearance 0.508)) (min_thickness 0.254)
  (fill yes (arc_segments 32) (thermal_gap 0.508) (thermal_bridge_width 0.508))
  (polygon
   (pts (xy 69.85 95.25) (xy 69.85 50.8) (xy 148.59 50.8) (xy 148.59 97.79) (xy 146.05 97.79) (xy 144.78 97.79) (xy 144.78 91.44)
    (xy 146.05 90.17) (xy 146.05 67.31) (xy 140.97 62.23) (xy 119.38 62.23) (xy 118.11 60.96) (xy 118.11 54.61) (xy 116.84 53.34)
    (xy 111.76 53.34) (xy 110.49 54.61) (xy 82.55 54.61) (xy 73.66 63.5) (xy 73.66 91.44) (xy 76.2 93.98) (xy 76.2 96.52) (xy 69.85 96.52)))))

